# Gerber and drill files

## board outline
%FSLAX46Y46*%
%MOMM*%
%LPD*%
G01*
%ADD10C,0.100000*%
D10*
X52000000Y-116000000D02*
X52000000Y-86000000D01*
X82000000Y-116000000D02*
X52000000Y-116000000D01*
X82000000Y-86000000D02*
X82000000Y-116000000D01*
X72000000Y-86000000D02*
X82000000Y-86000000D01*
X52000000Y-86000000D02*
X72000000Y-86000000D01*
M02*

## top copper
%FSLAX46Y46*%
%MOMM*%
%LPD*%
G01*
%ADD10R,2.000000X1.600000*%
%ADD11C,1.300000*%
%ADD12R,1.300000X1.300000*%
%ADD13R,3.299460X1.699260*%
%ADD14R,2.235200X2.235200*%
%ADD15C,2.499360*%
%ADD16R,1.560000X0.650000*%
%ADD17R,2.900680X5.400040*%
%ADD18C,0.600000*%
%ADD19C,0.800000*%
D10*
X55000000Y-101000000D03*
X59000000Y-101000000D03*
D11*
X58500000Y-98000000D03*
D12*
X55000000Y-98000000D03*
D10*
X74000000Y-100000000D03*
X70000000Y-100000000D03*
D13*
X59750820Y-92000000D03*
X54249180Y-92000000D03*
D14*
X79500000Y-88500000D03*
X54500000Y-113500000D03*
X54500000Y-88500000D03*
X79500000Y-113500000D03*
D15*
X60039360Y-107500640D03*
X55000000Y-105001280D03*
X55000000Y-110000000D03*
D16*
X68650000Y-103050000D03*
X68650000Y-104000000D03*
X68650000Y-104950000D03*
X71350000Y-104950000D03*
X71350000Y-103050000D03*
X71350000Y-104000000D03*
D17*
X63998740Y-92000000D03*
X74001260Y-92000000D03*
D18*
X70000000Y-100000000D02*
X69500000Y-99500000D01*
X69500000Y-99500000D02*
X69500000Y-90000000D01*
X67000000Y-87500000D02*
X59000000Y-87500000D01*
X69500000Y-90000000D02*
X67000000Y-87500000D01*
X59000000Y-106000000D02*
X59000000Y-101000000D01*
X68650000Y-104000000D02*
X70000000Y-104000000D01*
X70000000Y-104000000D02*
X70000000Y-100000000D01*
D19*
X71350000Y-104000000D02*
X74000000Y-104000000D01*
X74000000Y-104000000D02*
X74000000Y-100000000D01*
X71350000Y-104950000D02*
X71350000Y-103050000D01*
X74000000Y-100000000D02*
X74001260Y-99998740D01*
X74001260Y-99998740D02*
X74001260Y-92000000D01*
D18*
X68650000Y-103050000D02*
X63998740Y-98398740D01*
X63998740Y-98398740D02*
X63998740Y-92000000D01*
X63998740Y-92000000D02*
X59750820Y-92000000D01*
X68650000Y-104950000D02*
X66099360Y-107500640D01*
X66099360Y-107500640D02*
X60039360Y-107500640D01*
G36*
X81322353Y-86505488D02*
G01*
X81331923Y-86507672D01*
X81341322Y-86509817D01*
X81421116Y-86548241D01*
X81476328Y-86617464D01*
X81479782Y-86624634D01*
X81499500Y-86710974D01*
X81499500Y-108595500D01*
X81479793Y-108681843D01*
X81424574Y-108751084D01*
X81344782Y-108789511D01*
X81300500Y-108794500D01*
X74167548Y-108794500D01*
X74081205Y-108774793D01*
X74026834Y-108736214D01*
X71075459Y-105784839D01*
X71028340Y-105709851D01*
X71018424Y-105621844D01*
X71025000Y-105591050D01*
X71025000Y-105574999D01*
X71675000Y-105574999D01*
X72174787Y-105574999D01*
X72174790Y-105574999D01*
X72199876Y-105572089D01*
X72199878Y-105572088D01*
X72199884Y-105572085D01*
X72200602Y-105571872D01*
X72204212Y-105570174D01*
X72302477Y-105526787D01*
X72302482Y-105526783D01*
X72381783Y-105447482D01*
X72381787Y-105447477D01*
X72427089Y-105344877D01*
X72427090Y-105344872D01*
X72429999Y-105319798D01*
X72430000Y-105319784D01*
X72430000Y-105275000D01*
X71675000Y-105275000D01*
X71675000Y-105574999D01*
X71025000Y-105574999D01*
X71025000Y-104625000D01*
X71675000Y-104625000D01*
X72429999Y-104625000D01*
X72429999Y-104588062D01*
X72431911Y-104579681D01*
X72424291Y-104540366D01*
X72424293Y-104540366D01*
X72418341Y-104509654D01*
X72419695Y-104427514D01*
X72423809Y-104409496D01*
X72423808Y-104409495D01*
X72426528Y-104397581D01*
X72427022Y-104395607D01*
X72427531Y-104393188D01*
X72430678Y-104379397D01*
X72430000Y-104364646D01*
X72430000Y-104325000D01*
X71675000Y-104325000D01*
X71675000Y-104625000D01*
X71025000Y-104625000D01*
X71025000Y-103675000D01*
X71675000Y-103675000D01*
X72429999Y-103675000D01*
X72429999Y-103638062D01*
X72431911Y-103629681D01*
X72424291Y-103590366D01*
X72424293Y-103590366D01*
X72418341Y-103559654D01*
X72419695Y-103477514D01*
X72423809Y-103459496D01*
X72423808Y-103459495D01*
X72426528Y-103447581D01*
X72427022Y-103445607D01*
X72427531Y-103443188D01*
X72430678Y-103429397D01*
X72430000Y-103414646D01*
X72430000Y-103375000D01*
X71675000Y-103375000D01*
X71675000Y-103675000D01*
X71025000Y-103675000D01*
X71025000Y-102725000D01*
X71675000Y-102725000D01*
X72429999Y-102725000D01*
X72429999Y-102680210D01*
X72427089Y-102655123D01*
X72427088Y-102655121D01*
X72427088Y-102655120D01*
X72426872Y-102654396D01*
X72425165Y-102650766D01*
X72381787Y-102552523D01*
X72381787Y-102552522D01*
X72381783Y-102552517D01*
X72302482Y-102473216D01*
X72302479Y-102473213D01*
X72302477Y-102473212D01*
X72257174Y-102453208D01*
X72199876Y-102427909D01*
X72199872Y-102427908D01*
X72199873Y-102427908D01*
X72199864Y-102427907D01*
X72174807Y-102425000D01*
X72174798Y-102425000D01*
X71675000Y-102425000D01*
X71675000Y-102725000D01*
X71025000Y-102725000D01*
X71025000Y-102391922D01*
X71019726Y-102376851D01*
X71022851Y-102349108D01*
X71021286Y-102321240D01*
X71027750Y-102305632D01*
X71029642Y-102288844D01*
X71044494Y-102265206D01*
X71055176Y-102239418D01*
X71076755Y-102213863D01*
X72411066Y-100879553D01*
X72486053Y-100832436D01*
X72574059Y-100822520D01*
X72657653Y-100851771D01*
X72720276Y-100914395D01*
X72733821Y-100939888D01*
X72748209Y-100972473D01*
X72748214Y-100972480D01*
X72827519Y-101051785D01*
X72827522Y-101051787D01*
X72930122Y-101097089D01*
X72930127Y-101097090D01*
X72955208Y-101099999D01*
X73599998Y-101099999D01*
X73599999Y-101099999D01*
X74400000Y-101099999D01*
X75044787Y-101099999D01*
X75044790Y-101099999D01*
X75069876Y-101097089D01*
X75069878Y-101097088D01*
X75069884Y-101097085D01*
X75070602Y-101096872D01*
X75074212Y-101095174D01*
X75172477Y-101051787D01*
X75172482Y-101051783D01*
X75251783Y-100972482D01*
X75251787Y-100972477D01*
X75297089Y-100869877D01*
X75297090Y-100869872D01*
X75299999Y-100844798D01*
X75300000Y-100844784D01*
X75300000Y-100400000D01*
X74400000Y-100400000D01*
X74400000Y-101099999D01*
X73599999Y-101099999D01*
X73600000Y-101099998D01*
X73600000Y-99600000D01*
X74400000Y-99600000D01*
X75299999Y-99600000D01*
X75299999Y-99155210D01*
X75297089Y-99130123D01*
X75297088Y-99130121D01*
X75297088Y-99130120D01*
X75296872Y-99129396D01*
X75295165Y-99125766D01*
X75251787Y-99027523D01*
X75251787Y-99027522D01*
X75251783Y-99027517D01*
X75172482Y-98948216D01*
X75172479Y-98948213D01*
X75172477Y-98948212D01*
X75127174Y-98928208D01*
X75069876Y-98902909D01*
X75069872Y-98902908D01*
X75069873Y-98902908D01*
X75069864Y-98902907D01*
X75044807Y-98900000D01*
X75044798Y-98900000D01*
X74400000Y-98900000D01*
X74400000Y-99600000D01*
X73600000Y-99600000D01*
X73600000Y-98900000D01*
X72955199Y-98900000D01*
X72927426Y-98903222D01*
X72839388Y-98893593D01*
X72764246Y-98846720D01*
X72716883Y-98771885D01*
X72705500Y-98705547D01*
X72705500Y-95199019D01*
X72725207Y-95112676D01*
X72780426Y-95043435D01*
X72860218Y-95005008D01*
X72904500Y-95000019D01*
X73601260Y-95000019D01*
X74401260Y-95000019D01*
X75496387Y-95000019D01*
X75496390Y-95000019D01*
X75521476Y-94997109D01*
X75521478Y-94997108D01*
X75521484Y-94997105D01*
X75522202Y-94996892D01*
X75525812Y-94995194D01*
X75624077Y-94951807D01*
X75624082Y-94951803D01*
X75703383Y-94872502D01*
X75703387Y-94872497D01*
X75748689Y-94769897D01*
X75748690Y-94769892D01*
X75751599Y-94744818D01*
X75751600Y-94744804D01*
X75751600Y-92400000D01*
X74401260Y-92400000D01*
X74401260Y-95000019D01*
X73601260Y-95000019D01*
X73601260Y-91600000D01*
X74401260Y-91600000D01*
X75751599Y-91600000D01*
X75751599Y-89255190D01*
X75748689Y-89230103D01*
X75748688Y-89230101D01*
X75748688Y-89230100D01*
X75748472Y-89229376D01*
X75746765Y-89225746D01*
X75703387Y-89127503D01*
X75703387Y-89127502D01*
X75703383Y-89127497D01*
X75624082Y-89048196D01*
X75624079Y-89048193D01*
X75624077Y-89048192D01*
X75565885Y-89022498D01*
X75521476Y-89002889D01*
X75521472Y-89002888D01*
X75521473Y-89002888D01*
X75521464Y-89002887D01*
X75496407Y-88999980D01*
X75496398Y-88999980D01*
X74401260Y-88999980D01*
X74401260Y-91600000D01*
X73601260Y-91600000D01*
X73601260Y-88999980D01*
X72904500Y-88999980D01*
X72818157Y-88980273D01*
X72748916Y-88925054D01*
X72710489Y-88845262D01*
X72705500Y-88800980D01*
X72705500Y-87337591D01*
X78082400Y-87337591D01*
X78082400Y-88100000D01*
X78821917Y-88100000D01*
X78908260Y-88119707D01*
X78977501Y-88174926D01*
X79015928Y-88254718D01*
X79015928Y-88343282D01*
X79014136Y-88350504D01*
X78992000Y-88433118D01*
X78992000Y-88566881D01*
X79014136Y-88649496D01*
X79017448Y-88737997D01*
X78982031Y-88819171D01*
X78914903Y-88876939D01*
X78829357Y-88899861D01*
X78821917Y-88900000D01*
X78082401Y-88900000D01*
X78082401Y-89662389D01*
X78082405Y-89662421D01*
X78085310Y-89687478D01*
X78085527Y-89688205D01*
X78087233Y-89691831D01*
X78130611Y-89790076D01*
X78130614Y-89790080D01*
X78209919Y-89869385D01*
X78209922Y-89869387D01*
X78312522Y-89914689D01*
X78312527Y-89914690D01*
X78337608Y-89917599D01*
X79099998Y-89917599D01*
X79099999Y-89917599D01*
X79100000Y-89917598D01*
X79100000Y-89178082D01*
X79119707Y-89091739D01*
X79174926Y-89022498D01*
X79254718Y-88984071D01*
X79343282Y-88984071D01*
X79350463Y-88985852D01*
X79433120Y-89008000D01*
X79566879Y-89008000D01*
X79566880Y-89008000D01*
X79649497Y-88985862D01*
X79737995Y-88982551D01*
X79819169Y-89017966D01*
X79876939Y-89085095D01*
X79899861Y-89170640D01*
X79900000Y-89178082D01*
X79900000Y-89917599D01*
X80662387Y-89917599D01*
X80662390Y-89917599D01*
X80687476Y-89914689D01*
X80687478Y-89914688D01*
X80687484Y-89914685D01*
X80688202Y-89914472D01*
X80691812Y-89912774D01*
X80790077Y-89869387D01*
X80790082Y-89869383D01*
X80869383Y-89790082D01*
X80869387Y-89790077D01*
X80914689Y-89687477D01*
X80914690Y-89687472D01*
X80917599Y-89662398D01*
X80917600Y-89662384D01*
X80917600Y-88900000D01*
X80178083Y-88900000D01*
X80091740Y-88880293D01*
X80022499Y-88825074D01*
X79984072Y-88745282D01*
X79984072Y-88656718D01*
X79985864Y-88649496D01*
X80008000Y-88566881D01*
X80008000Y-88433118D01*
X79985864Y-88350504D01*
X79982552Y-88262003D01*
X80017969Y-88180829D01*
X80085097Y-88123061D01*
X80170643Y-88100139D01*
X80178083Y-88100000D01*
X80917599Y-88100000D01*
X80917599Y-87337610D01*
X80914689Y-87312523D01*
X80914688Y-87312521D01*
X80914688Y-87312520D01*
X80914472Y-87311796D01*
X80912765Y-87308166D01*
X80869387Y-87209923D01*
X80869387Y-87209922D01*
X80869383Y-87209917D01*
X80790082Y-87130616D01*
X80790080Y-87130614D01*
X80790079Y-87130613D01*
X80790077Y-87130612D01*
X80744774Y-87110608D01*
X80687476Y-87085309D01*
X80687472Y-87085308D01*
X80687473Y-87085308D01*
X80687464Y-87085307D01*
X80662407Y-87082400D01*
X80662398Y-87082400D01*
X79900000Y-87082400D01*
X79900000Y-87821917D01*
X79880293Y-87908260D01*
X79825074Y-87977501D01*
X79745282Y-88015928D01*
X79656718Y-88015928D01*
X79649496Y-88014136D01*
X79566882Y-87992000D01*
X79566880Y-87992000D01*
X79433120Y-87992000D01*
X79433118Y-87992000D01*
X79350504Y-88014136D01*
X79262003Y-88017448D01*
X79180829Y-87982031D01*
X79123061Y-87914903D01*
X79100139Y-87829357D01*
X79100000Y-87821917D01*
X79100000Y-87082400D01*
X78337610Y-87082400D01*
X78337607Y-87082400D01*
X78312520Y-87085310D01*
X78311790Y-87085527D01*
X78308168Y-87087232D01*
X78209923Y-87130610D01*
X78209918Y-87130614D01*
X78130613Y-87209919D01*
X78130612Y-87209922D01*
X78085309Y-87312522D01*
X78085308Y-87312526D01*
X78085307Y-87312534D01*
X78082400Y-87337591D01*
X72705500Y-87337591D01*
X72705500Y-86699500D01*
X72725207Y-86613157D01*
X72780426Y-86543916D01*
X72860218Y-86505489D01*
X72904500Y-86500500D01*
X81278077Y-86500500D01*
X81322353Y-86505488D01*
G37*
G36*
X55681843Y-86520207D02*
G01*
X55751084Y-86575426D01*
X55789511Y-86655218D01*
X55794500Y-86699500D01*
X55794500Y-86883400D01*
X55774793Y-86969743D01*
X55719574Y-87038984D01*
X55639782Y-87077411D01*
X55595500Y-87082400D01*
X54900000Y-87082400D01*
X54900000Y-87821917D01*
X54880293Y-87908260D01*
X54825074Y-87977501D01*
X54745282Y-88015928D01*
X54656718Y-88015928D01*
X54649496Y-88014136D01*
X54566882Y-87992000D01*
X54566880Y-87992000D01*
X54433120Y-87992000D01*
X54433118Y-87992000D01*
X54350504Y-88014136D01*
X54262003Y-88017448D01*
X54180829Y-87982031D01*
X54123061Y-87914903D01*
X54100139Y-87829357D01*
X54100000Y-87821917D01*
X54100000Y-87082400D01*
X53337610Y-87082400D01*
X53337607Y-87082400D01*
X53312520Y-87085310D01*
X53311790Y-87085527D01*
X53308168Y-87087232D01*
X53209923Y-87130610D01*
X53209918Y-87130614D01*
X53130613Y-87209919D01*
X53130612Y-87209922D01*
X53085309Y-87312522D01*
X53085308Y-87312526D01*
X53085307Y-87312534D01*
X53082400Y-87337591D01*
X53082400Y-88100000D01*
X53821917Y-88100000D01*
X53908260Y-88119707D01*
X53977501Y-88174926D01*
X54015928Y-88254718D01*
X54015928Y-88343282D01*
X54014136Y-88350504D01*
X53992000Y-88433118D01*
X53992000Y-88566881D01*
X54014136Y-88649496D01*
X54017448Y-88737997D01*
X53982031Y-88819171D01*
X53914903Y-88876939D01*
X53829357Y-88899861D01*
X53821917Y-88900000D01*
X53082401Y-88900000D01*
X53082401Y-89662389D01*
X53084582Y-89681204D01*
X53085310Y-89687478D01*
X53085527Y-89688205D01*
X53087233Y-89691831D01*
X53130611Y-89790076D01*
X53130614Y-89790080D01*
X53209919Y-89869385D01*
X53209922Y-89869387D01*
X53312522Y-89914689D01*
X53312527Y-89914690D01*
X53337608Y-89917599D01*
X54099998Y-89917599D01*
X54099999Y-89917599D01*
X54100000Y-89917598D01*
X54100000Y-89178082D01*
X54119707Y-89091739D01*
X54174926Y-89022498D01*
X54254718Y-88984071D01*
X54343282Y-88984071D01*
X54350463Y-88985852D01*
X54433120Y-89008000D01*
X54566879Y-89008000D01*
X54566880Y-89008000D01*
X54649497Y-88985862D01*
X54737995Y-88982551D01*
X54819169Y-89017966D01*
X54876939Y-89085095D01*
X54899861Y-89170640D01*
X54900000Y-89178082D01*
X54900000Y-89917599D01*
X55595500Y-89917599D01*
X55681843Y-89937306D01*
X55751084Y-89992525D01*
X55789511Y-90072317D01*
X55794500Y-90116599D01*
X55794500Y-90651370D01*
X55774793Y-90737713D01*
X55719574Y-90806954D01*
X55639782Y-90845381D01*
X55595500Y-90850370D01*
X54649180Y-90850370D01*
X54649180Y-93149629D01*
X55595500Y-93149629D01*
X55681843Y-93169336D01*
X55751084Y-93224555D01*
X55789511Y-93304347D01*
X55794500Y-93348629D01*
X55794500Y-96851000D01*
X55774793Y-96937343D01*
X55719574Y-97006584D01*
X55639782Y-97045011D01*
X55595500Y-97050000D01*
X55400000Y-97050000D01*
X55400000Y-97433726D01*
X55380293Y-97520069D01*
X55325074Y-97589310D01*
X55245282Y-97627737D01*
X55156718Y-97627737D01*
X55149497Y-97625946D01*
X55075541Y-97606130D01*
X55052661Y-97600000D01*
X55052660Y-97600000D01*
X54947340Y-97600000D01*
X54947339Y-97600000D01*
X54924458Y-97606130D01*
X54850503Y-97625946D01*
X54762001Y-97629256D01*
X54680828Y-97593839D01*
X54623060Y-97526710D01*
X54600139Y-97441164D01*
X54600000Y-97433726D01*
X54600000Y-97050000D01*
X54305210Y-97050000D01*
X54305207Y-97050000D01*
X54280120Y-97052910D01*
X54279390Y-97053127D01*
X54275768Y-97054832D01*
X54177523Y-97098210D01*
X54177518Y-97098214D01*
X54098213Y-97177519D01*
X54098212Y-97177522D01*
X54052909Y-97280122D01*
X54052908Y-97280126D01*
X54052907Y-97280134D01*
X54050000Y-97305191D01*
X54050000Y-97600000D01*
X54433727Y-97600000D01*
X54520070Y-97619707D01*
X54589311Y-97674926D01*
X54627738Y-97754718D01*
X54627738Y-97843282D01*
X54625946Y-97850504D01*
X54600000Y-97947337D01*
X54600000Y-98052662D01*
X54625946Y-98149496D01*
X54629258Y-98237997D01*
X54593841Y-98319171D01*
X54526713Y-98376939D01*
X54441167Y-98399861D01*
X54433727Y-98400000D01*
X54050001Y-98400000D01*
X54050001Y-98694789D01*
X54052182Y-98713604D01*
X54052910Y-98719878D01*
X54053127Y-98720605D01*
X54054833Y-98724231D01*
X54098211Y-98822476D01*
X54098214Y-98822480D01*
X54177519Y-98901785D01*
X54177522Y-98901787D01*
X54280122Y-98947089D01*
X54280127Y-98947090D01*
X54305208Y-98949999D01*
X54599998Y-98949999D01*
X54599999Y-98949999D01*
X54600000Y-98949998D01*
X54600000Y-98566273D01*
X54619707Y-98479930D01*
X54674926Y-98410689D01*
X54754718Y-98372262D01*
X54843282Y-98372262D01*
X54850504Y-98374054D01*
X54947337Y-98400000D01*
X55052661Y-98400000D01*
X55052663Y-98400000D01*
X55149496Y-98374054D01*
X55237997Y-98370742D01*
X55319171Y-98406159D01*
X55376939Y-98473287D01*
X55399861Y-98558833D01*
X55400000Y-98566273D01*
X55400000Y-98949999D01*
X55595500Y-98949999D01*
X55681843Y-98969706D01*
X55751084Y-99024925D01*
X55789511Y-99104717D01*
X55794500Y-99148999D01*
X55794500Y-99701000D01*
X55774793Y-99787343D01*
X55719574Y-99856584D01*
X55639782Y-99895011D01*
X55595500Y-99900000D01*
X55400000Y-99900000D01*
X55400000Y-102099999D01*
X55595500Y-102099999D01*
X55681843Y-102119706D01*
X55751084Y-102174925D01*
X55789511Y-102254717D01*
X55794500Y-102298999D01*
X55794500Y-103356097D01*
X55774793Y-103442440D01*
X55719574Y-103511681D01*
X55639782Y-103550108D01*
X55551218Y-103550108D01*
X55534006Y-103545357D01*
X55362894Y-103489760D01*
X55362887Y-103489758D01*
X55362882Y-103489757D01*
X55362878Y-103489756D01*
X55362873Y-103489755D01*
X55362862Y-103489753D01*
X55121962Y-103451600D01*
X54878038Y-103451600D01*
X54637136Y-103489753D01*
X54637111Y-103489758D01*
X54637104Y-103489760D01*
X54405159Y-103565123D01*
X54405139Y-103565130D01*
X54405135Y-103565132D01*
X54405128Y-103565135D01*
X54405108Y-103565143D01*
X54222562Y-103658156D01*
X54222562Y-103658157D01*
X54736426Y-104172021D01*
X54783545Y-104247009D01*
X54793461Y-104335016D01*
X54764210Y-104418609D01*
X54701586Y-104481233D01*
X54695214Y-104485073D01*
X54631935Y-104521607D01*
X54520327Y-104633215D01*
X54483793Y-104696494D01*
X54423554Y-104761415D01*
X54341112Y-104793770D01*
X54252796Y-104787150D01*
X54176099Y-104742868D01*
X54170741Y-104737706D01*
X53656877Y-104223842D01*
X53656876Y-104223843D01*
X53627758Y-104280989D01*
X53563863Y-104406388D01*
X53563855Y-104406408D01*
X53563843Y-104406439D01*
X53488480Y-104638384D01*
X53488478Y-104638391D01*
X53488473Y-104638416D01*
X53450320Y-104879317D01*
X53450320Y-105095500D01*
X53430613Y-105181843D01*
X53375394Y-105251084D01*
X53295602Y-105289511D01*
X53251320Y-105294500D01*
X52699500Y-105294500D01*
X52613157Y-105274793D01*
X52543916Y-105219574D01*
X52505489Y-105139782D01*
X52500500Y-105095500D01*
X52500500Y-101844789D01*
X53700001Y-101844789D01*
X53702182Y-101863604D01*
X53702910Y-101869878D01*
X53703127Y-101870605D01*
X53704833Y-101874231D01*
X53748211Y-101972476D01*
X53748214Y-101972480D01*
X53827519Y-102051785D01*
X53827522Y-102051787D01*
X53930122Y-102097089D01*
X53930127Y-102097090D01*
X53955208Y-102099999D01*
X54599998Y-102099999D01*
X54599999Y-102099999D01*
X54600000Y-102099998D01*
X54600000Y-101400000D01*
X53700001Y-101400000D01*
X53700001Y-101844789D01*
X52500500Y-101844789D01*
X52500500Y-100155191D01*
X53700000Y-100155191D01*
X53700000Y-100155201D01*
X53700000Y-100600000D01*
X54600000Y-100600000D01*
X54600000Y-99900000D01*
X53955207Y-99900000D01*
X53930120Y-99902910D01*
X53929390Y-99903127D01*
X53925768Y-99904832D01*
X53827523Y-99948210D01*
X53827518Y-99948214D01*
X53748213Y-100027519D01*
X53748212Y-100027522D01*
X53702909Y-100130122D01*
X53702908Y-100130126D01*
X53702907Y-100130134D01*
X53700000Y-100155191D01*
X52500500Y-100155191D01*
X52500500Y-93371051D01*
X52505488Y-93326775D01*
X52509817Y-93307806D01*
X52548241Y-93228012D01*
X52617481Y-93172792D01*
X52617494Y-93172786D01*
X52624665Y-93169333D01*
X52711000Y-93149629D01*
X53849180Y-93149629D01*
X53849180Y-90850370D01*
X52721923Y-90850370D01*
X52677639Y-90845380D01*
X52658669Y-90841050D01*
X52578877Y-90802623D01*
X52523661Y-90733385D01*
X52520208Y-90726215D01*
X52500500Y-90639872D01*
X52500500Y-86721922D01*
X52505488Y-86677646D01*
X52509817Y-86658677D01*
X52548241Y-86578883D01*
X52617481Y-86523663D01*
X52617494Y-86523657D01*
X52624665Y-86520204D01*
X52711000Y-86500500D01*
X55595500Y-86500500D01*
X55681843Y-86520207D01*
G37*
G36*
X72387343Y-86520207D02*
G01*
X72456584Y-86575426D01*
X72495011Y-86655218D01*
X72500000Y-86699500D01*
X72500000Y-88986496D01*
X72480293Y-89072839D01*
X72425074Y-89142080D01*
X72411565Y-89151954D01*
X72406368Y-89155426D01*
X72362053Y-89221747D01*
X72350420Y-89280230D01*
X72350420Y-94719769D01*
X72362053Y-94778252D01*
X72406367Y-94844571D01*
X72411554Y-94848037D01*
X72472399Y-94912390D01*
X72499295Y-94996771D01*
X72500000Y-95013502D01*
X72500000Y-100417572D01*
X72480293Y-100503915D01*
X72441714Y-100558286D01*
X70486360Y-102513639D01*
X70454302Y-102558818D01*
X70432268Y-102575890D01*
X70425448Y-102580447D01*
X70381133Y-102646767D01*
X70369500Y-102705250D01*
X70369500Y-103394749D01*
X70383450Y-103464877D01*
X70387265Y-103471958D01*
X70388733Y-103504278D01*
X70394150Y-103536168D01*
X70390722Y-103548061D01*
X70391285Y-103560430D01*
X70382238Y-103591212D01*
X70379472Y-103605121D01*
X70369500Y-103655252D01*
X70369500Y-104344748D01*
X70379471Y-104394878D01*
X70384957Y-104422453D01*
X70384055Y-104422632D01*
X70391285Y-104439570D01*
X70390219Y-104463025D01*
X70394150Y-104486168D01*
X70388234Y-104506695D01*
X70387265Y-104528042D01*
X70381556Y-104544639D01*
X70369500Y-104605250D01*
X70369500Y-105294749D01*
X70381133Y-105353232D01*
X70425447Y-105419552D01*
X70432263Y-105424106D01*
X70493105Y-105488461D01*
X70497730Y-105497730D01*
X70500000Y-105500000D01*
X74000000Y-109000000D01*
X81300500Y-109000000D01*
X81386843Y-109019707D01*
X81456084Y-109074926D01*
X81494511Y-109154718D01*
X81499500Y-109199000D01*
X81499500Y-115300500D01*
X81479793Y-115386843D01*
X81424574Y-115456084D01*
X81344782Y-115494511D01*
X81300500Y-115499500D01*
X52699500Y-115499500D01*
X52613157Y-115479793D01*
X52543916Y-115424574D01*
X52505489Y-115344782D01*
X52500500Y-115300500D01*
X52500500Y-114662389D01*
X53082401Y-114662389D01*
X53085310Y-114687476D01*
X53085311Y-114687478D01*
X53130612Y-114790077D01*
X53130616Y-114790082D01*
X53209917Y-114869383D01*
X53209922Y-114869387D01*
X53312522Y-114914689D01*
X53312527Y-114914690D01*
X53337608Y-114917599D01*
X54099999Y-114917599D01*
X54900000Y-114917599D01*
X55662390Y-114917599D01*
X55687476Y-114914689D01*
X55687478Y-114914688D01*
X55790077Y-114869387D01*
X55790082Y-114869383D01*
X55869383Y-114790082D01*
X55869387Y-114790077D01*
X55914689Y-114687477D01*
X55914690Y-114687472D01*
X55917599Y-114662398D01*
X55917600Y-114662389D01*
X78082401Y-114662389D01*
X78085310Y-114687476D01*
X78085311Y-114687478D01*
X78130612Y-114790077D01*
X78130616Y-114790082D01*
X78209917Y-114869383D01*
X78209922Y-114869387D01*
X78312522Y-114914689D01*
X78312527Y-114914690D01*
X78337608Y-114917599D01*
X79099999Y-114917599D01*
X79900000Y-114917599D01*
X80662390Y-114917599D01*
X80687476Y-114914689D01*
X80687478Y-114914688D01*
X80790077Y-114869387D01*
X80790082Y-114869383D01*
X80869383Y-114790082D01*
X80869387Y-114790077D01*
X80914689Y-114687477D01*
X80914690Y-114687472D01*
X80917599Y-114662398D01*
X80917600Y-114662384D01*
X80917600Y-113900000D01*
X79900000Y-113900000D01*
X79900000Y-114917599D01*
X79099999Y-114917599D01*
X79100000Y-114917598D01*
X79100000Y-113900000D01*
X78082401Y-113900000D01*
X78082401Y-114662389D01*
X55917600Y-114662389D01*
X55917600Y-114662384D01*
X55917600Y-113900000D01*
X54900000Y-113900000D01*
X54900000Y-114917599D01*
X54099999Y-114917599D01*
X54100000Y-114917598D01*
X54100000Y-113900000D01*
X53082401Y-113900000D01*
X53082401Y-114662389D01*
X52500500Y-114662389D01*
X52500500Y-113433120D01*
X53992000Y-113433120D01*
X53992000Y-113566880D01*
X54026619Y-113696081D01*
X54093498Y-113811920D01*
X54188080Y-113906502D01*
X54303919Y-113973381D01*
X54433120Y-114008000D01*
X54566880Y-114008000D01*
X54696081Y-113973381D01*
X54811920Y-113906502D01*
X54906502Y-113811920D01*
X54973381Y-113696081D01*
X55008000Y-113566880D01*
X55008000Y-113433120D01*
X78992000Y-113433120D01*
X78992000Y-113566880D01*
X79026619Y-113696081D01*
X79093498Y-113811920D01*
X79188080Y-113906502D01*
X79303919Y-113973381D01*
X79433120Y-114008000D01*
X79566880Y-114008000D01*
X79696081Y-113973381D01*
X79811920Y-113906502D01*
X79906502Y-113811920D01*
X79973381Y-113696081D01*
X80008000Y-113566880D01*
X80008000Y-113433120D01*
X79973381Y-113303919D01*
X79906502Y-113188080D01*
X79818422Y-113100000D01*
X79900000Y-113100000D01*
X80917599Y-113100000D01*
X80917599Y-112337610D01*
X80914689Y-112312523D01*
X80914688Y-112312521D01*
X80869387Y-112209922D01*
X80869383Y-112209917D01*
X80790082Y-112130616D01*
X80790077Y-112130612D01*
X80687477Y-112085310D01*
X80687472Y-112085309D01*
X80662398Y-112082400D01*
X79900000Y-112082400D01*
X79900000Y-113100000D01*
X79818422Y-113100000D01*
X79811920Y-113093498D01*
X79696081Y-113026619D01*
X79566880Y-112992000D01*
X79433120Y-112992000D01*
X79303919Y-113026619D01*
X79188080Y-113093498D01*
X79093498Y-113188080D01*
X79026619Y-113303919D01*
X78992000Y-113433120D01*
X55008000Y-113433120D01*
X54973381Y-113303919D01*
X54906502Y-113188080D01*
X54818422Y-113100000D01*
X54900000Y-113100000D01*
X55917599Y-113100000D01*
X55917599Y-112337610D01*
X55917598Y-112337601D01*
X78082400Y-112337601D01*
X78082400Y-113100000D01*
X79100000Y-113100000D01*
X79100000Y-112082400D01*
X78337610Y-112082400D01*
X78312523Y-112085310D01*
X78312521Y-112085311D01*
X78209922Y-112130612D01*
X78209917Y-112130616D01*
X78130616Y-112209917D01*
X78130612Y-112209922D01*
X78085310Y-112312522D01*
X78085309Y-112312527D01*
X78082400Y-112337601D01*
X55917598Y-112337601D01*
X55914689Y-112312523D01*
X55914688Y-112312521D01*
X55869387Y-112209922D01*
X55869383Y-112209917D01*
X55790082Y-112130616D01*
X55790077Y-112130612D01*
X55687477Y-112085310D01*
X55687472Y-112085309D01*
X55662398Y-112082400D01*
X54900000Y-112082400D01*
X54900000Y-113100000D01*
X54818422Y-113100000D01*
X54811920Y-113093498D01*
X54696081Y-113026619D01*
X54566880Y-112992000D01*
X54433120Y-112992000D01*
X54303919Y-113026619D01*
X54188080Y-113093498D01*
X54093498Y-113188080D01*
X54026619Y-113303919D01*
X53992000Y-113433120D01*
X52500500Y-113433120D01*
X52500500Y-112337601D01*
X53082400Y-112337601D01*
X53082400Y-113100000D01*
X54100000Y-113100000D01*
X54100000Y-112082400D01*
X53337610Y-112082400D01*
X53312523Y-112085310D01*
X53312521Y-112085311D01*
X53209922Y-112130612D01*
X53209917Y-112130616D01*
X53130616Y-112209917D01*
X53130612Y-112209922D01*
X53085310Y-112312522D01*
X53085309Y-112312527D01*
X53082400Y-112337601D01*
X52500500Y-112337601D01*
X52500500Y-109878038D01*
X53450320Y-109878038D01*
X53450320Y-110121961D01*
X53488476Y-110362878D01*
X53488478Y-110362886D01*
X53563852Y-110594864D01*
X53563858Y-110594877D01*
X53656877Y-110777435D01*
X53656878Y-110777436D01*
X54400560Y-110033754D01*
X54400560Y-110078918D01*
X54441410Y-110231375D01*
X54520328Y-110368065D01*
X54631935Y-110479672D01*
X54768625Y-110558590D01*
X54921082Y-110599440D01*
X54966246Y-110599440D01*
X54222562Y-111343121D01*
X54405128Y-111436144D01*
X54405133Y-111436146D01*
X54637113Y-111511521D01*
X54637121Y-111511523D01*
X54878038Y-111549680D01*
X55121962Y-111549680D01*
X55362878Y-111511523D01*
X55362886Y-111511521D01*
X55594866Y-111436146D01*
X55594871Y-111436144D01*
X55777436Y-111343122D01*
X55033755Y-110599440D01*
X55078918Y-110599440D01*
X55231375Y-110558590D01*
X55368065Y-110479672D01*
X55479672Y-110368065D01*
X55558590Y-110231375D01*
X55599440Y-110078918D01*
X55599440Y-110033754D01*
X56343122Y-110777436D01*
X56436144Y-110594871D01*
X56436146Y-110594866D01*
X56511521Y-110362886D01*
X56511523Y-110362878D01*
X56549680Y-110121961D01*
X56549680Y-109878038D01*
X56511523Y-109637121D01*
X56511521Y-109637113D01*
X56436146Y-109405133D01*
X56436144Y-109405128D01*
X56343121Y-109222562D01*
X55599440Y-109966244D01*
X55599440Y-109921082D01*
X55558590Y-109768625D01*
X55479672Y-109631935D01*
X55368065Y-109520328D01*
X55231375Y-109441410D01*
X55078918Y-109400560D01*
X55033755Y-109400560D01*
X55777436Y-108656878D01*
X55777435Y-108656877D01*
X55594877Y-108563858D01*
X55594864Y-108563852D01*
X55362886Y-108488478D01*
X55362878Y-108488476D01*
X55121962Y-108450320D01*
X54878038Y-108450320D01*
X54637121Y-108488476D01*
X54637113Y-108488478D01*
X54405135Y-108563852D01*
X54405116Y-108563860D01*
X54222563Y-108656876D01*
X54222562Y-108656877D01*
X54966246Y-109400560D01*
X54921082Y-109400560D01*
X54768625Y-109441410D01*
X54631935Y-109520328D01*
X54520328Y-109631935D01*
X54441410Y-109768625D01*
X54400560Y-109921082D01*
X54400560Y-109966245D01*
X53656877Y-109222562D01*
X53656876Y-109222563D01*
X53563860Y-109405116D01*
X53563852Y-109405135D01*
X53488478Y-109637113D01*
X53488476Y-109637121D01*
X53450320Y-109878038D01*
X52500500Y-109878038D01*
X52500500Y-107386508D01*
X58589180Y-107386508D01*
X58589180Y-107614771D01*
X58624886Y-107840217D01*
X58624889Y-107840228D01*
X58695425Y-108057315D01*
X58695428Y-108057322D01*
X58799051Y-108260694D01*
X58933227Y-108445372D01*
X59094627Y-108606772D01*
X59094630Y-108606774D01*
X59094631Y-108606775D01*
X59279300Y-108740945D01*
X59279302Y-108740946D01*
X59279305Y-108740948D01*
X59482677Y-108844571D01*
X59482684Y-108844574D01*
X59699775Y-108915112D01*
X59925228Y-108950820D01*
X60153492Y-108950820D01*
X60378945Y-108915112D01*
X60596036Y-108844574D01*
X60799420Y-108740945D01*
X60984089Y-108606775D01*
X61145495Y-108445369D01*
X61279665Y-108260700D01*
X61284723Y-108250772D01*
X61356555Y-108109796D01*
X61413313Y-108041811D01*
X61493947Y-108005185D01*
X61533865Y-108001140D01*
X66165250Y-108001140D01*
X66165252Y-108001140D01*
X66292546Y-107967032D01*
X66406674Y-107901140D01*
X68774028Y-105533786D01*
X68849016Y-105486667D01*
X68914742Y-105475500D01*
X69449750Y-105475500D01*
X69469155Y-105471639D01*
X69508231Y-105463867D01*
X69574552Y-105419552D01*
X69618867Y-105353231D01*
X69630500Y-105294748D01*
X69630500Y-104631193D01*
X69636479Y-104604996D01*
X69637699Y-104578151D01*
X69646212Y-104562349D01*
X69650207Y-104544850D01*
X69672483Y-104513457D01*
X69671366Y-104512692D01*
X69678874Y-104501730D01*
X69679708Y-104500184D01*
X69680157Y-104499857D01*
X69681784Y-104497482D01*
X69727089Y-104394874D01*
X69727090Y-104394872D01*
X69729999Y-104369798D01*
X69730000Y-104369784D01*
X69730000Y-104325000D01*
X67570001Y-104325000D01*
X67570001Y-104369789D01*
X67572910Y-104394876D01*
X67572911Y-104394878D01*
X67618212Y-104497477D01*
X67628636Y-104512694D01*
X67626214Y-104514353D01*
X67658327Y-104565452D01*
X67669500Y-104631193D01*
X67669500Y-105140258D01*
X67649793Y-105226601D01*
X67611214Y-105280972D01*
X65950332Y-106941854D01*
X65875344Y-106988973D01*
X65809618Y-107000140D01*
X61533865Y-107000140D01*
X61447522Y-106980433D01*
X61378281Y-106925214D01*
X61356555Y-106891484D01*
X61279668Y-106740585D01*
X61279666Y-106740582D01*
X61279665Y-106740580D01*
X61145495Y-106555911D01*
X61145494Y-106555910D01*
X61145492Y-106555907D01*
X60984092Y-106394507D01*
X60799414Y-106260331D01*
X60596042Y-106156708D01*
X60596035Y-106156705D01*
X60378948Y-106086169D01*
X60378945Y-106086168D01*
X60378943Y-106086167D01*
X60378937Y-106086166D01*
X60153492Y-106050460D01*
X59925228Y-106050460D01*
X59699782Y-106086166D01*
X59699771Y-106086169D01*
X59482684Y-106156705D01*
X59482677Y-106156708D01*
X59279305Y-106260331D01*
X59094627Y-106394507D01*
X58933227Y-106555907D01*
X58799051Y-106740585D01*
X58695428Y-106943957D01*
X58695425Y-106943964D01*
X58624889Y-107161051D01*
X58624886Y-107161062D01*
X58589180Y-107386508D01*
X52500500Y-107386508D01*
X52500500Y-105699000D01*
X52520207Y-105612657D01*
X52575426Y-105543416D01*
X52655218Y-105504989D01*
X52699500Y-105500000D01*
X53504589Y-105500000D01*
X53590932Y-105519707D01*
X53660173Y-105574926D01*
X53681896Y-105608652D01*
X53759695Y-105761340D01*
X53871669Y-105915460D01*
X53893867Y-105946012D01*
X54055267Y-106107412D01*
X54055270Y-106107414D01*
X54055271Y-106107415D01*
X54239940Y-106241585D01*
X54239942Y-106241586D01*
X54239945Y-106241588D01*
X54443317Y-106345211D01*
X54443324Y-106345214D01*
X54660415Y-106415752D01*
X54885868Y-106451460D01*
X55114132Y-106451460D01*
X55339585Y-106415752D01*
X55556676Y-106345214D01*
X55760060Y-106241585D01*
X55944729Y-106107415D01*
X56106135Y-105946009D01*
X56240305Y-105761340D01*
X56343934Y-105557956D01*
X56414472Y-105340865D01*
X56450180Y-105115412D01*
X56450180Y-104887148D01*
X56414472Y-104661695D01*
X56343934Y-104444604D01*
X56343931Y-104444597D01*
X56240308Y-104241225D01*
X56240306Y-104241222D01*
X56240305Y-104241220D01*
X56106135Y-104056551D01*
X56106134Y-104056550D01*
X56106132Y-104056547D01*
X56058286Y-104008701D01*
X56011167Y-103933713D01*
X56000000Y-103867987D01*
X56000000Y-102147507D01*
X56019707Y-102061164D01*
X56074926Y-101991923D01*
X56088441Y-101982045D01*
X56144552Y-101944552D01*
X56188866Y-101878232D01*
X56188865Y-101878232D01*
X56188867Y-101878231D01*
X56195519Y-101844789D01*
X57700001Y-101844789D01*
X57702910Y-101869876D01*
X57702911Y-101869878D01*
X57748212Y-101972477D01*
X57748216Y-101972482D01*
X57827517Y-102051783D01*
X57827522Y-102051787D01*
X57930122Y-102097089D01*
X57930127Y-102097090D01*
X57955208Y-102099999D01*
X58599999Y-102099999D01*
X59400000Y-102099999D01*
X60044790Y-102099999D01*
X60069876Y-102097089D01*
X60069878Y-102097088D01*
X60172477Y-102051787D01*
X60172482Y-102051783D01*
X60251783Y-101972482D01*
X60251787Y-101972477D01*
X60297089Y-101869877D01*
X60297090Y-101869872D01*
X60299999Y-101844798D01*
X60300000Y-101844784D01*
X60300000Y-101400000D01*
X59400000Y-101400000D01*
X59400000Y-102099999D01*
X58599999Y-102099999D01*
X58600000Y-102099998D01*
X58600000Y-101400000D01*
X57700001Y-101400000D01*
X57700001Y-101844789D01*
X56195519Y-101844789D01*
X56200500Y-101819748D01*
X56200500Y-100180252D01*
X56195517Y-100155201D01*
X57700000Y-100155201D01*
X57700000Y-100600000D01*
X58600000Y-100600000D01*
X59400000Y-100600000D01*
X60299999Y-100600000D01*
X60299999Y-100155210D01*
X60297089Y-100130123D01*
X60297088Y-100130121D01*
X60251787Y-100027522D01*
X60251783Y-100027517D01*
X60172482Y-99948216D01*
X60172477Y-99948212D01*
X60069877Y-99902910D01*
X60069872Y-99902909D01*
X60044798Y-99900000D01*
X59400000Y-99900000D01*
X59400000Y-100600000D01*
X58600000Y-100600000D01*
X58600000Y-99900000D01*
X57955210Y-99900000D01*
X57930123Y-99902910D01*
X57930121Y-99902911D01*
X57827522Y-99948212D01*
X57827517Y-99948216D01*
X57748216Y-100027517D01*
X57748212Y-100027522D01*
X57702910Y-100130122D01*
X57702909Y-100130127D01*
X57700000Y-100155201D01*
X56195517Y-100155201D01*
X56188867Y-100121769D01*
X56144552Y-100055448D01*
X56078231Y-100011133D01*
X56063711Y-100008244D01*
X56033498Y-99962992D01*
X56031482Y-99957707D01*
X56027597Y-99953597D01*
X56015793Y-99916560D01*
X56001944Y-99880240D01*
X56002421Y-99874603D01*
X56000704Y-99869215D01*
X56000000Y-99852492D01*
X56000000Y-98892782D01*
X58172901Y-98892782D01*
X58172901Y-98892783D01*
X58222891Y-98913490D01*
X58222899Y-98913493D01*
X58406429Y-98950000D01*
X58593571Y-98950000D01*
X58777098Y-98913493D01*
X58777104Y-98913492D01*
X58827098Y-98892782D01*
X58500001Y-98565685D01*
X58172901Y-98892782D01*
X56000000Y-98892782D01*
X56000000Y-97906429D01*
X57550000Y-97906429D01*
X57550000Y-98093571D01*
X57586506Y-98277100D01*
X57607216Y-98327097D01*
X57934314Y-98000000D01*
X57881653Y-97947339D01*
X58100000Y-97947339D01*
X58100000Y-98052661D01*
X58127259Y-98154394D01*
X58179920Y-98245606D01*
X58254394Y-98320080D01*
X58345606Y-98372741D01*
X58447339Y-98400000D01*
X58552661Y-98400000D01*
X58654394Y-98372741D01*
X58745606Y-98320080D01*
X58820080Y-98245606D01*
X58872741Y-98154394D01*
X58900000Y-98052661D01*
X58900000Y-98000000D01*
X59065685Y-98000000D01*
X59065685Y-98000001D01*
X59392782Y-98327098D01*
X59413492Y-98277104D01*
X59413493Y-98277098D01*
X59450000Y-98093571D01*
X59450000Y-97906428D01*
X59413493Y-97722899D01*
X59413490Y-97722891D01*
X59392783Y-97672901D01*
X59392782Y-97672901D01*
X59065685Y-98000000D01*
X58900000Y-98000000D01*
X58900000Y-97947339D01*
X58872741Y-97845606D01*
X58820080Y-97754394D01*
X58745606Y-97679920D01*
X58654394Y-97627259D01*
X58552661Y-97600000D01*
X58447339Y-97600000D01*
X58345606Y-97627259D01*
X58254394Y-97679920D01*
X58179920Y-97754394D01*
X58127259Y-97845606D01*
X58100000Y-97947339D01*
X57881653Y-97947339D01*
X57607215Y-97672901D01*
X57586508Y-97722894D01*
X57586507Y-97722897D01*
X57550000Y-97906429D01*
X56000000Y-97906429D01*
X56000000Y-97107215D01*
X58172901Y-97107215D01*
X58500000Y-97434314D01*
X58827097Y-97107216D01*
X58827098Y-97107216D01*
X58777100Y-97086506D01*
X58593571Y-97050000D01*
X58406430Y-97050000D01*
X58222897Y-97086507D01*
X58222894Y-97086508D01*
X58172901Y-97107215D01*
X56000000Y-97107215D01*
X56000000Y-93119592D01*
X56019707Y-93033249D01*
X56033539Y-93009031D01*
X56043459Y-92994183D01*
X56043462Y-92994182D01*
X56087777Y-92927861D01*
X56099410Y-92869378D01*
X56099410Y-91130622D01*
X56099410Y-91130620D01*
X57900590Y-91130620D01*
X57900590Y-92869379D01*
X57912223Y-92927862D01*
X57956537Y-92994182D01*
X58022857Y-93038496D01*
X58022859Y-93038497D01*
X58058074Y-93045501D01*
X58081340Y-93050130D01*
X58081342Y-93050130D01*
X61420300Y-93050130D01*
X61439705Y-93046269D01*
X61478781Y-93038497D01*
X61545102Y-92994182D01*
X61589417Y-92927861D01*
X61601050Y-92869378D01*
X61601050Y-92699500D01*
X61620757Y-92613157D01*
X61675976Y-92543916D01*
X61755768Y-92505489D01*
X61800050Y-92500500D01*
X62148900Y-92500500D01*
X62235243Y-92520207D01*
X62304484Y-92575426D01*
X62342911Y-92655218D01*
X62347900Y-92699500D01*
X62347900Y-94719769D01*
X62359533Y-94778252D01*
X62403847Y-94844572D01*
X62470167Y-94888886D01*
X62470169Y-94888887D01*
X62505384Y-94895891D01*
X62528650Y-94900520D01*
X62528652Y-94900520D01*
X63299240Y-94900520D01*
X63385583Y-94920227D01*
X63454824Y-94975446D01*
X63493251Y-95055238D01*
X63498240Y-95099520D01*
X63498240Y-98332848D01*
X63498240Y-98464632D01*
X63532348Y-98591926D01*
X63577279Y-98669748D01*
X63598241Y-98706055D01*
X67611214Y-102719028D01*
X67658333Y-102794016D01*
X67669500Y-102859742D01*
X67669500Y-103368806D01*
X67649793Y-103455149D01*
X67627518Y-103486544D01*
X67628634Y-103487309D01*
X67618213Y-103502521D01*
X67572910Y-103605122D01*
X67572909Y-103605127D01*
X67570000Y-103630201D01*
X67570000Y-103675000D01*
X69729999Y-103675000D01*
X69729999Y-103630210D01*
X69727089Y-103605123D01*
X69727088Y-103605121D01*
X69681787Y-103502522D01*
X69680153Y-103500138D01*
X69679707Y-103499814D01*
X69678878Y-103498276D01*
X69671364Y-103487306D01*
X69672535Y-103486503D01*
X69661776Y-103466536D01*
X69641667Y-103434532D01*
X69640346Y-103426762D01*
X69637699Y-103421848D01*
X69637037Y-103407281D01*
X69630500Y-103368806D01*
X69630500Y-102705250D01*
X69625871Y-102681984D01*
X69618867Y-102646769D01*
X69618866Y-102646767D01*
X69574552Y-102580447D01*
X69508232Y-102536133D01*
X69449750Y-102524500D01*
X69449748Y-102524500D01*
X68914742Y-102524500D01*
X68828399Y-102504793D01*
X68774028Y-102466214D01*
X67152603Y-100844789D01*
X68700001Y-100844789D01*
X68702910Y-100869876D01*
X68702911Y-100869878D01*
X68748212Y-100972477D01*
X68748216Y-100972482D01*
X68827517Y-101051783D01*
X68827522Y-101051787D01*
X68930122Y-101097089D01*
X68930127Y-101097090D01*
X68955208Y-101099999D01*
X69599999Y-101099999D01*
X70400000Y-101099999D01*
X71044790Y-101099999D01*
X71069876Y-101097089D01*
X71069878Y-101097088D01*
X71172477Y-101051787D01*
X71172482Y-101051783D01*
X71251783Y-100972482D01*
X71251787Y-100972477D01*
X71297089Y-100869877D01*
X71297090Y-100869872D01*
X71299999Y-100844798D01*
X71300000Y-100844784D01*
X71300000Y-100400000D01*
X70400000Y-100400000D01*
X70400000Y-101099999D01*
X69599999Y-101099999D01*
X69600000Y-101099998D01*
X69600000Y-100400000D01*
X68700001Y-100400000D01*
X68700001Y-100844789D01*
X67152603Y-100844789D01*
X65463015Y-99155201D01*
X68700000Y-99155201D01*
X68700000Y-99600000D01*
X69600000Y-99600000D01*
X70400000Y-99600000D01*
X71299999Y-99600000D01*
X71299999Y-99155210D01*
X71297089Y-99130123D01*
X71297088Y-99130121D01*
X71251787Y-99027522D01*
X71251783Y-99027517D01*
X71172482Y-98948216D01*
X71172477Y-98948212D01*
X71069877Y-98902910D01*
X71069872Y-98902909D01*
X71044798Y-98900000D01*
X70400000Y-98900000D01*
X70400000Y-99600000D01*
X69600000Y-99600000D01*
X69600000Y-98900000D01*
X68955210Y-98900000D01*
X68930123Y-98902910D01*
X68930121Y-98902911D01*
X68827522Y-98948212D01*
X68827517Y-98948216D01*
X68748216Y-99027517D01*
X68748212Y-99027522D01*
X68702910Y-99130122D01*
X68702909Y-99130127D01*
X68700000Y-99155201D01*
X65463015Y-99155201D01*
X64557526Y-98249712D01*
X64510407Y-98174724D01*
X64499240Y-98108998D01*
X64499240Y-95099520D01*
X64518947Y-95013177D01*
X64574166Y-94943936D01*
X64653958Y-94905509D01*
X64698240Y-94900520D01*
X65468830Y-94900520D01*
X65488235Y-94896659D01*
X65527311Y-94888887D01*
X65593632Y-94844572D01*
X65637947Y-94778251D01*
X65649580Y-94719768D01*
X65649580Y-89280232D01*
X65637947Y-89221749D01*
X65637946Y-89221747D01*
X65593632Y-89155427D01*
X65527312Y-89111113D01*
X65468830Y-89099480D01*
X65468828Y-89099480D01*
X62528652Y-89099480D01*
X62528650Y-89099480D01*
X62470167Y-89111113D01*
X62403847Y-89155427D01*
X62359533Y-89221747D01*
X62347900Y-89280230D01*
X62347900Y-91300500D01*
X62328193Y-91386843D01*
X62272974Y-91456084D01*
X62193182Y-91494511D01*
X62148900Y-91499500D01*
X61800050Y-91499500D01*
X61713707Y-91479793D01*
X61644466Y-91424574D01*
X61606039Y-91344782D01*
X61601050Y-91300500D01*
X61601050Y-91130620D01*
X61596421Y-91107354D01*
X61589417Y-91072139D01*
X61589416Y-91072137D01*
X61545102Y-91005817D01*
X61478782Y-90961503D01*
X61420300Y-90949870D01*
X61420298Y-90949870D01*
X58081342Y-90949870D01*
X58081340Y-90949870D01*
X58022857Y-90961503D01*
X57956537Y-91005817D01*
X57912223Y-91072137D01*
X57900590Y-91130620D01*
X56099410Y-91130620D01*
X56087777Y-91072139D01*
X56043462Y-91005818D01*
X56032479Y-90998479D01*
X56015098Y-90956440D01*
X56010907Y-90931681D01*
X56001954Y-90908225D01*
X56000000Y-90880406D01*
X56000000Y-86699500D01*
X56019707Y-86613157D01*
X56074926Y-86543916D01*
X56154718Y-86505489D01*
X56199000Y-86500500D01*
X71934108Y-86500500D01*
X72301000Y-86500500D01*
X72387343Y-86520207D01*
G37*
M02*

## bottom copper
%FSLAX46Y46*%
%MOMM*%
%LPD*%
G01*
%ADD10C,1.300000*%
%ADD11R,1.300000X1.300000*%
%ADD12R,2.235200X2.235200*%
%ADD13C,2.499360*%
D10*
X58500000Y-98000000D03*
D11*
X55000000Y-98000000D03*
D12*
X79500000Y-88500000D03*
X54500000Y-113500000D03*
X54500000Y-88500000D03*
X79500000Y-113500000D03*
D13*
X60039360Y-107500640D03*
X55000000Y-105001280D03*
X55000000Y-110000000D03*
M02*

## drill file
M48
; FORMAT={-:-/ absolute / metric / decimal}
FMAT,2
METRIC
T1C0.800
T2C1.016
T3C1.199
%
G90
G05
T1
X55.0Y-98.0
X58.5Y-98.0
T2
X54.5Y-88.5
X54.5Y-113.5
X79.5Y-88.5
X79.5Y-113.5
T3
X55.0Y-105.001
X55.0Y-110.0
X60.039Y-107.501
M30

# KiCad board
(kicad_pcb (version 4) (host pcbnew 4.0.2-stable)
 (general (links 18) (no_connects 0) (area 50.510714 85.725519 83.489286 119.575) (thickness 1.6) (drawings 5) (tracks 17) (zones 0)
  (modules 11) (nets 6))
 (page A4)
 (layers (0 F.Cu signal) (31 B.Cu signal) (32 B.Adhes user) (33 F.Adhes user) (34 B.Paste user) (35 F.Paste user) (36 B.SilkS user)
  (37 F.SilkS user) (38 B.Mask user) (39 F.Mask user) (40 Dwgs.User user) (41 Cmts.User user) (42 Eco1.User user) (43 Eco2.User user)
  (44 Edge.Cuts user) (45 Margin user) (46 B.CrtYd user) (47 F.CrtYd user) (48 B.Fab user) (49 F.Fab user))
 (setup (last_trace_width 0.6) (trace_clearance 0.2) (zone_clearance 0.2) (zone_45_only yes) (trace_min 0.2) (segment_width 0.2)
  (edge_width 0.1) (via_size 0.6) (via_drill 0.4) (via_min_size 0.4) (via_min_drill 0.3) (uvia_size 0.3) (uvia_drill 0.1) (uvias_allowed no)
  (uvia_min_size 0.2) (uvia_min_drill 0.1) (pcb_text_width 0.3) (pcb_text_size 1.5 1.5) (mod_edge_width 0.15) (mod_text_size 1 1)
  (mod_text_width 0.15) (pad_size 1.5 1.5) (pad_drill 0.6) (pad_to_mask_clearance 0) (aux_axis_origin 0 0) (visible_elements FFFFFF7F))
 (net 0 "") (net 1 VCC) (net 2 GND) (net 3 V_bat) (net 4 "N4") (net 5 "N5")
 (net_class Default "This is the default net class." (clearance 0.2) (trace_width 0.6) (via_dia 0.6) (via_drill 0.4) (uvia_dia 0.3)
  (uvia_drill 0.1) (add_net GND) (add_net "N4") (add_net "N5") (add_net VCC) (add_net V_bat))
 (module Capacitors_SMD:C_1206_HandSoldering (layer F.Cu) (at 57 101)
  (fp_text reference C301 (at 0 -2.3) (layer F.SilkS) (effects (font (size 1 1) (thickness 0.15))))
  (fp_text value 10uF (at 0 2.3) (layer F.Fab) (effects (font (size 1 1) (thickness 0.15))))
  (pad 1 smd rect (at -2 0) (size 2 1.6) (layers F.Cu F.Paste F.Mask) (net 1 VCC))
  (pad 2 smd rect (at 2 0) (size 2 1.6) (layers F.Cu F.Paste F.Mask) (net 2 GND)))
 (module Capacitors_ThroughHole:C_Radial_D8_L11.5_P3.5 (layer B.Cu) (at 55 98)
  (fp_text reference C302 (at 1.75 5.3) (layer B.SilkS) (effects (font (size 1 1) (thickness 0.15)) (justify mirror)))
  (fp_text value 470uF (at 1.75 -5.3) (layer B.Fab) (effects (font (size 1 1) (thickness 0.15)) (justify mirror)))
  (pad 2 thru_hole circle (at 3.5 0) (size 1.3 1.3) (drill 0.8) (layers *.Cu *.Mask B.SilkS) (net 2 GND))
  (pad 1 thru_hole rect (at 0 0) (size 1.3 1.3) (drill 0.8) (layers *.Cu *.Mask B.SilkS) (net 1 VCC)))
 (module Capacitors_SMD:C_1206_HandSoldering (layer F.Cu) (at 72 100 180)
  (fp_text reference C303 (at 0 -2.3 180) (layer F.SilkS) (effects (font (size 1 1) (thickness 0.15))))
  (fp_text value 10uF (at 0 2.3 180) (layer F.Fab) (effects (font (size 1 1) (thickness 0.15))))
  (pad 1 smd rect (at -2 0 180) (size 2 1.6) (layers F.Cu F.Paste F.Mask) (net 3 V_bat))
  (pad 2 smd rect (at 2 0 180) (size 2 1.6) (layers F.Cu F.Paste F.Mask) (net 2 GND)))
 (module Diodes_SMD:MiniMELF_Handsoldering (layer F.Cu) (at 57 92 180)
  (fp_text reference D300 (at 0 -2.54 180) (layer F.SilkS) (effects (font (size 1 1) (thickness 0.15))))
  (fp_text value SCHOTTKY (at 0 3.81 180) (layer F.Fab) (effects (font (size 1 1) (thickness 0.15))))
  (pad 1 smd rect (at -2.75082 0 180) (size 3.29946 1.69926) (layers F.Cu F.Paste F.Mask) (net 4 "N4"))
  (pad 2 smd rect (at 2.75082 0 180) (size 3.29946 1.69926) (layers F.Cu F.Paste F.Mask) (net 1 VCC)))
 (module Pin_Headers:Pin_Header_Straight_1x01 (layer B.Cu) (at 79.5 88.5)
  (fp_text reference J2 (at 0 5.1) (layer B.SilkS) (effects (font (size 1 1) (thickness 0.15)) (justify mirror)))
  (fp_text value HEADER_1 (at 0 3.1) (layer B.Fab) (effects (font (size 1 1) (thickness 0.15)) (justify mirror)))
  (pad 1 thru_hole rect (at 0 0) (size 2.2352 2.2352) (drill 1.016) (layers *.Cu *.Mask B.SilkS) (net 3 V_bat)))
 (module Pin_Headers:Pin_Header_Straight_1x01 (layer B.Cu) (at 54.5 113.5)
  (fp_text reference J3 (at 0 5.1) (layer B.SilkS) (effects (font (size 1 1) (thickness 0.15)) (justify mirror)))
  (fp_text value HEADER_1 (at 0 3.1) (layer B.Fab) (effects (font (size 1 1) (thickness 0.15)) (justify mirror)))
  (pad 1 thru_hole rect (at 0 0) (size 2.2352 2.2352) (drill 1.016) (layers *.Cu *.Mask B.SilkS) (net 2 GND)))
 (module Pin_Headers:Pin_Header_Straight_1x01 (layer B.Cu) (at 54.5 88.5)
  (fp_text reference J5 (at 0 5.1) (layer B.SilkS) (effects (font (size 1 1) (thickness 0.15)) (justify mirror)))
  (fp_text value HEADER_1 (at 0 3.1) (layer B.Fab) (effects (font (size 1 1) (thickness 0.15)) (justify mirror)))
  (pad 1 thru_hole rect (at 0 0) (size 2.2352 2.2352) (drill 1.016) (layers *.Cu *.Mask B.SilkS) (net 1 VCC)))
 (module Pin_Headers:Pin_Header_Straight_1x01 (layer B.Cu) (at 79.5 113.5)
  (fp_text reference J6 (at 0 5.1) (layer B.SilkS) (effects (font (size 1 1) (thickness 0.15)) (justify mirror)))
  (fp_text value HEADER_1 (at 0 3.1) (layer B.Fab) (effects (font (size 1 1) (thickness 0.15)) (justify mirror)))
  (pad 1 thru_hole rect (at 0 0) (size 2.2352 2.2352) (drill 1.016) (layers *.Cu *.Mask B.SilkS) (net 2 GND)))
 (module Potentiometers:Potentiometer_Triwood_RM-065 (layer B.Cu) (at 55 110 90)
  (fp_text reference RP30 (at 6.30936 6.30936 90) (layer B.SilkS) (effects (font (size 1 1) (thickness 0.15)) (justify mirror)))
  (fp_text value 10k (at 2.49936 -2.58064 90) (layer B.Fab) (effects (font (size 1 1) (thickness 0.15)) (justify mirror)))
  (pad 2 thru_hole circle (at 2.49936 5.03936 90) (size 2.49936 2.49936) (drill 1.19888) (layers *.Cu *.Mask B.SilkS) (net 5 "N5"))
  (pad 3 thru_hole circle (at 4.99872 0 90) (size 2.49936 2.49936) (drill 1.19888) (layers *.Cu *.Mask B.SilkS) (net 1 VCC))
  (pad 1 thru_hole circle (at 0 0 90) (size 2.49936 2.49936) (drill 1.19888) (layers *.Cu *.Mask B.SilkS) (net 2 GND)))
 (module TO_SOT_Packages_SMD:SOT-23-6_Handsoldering (layer F.Cu) (at 70 104)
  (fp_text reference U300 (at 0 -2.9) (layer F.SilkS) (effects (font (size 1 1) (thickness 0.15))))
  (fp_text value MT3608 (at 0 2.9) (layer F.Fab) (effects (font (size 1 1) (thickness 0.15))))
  (pad 1 smd rect (at -1.35 -0.95) (size 1.56 0.65) (layers F.Cu F.Paste F.Mask) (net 4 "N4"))
  (pad 2 smd rect (at -1.35 0) (size 1.56 0.65) (layers F.Cu F.Paste F.Mask) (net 2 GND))
  (pad 3 smd rect (at -1.35 0.95) (size 1.56 0.65) (layers F.Cu F.Paste F.Mask) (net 5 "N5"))
  (pad 4 smd rect (at 1.35 0.95) (size 1.56 0.65) (layers F.Cu F.Paste F.Mask) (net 3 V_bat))
  (pad 6 smd rect (at 1.35 -0.95) (size 1.56 0.65) (layers F.Cu F.Paste F.Mask) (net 3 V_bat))
  (pad 5 smd rect (at 1.35 0) (size 1.56 0.65) (layers F.Cu F.Paste F.Mask) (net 3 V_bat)))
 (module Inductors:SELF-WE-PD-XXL (layer F.Cu) (at 69 92)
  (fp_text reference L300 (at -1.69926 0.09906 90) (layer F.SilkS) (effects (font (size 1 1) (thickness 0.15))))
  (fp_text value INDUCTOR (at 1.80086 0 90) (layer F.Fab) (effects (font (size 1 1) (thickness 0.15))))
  (pad 1 smd rect (at -5.00126 0) (size 2.90068 5.40004) (layers F.Cu F.Paste F.Mask) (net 4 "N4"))
  (pad 2 smd rect (at 5.00126 0) (size 2.90068 5.40004) (layers F.Cu F.Paste F.Mask) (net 3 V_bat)))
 (gr_line (start 52 116) (end 52 86) (angle 90) (layer Edge.Cuts) (width 0.1))
 (gr_line (start 82 116) (end 52 116) (angle 90) (layer Edge.Cuts) (width 0.1))
 (gr_line (start 82 86) (end 82 116) (angle 90) (layer Edge.Cuts) (width 0.1))
 (gr_line (start 72 86) (end 82 86) (angle 90) (layer Edge.Cuts) (width 0.1))
 (gr_line (start 52 86) (end 72 86) (angle 90) (layer Edge.Cuts) (width 0.1))
 (segment (start 70 100) (end 69.5 99.5) (width 0.6) (layer F.Cu) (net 2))
 (segment (start 69.5 99.5) (end 69.5 90) (width 0.6) (layer F.Cu) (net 2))
 (segment (start 67 87.5) (end 59 87.5) (width 0.6) (layer F.Cu) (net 2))
 (segment (start 69.5 90) (end 67 87.5) (width 0.6) (layer F.Cu) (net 2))
 (segment (start 59 106) (end 59 101) (width 0.6) (layer F.Cu) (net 2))
 (segment (start 68.65 104) (end 70 104) (width 0.6) (layer F.Cu) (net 2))
 (segment (start 70 104) (end 70 100) (width 0.6) (layer F.Cu) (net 2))
 (segment (start 71.35 104) (end 74 104) (width 0.8) (layer F.Cu) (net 3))
 (segment (start 74 104) (end 74 100) (width 0.8) (layer F.Cu) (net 3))
 (segment (start 71.35 104.95) (end 71.35 103.05) (width 0.8) (layer F.Cu) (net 3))
 (segment (start 74 100) (end 74.00126 99.99874) (width 0.8) (layer F.Cu) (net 3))
 (segment (start 74.00126 99.99874) (end 74.00126 92) (width 0.8) (layer F.Cu) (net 3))
 (segment (start 68.65 103.05) (end 63.99874 98.39874) (width 0.6) (layer F.Cu) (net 4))
 (segment (start 63.99874 98.39874) (end 63.99874 92) (width 0.6) (layer F.Cu) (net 4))
 (segment (start 63.99874 92) (end 59.75082 92) (width 0.6) (layer F.Cu) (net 4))
 (segment (start 68.65 104.95) (end 66.09936 107.50064) (width 0.6) (layer F.Cu) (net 5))
 (segment (start 66.09936 107.50064) (end 60.03936 107.50064) (width 0.6) (layer F.Cu) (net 5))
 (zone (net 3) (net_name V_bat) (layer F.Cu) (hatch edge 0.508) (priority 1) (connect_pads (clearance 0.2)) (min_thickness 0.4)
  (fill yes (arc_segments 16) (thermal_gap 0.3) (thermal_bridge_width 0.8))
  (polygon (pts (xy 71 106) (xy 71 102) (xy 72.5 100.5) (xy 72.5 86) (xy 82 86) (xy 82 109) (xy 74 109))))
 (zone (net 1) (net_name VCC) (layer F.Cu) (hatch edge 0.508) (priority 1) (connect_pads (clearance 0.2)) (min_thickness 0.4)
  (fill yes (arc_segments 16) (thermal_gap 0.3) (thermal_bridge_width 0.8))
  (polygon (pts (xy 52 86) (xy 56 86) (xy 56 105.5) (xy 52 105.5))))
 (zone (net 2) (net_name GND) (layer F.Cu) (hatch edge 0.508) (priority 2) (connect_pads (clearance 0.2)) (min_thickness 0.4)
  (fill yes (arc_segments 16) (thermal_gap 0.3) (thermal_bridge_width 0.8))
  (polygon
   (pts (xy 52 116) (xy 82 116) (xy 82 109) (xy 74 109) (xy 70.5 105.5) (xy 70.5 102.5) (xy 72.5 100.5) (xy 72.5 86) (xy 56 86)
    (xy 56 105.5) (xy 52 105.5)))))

